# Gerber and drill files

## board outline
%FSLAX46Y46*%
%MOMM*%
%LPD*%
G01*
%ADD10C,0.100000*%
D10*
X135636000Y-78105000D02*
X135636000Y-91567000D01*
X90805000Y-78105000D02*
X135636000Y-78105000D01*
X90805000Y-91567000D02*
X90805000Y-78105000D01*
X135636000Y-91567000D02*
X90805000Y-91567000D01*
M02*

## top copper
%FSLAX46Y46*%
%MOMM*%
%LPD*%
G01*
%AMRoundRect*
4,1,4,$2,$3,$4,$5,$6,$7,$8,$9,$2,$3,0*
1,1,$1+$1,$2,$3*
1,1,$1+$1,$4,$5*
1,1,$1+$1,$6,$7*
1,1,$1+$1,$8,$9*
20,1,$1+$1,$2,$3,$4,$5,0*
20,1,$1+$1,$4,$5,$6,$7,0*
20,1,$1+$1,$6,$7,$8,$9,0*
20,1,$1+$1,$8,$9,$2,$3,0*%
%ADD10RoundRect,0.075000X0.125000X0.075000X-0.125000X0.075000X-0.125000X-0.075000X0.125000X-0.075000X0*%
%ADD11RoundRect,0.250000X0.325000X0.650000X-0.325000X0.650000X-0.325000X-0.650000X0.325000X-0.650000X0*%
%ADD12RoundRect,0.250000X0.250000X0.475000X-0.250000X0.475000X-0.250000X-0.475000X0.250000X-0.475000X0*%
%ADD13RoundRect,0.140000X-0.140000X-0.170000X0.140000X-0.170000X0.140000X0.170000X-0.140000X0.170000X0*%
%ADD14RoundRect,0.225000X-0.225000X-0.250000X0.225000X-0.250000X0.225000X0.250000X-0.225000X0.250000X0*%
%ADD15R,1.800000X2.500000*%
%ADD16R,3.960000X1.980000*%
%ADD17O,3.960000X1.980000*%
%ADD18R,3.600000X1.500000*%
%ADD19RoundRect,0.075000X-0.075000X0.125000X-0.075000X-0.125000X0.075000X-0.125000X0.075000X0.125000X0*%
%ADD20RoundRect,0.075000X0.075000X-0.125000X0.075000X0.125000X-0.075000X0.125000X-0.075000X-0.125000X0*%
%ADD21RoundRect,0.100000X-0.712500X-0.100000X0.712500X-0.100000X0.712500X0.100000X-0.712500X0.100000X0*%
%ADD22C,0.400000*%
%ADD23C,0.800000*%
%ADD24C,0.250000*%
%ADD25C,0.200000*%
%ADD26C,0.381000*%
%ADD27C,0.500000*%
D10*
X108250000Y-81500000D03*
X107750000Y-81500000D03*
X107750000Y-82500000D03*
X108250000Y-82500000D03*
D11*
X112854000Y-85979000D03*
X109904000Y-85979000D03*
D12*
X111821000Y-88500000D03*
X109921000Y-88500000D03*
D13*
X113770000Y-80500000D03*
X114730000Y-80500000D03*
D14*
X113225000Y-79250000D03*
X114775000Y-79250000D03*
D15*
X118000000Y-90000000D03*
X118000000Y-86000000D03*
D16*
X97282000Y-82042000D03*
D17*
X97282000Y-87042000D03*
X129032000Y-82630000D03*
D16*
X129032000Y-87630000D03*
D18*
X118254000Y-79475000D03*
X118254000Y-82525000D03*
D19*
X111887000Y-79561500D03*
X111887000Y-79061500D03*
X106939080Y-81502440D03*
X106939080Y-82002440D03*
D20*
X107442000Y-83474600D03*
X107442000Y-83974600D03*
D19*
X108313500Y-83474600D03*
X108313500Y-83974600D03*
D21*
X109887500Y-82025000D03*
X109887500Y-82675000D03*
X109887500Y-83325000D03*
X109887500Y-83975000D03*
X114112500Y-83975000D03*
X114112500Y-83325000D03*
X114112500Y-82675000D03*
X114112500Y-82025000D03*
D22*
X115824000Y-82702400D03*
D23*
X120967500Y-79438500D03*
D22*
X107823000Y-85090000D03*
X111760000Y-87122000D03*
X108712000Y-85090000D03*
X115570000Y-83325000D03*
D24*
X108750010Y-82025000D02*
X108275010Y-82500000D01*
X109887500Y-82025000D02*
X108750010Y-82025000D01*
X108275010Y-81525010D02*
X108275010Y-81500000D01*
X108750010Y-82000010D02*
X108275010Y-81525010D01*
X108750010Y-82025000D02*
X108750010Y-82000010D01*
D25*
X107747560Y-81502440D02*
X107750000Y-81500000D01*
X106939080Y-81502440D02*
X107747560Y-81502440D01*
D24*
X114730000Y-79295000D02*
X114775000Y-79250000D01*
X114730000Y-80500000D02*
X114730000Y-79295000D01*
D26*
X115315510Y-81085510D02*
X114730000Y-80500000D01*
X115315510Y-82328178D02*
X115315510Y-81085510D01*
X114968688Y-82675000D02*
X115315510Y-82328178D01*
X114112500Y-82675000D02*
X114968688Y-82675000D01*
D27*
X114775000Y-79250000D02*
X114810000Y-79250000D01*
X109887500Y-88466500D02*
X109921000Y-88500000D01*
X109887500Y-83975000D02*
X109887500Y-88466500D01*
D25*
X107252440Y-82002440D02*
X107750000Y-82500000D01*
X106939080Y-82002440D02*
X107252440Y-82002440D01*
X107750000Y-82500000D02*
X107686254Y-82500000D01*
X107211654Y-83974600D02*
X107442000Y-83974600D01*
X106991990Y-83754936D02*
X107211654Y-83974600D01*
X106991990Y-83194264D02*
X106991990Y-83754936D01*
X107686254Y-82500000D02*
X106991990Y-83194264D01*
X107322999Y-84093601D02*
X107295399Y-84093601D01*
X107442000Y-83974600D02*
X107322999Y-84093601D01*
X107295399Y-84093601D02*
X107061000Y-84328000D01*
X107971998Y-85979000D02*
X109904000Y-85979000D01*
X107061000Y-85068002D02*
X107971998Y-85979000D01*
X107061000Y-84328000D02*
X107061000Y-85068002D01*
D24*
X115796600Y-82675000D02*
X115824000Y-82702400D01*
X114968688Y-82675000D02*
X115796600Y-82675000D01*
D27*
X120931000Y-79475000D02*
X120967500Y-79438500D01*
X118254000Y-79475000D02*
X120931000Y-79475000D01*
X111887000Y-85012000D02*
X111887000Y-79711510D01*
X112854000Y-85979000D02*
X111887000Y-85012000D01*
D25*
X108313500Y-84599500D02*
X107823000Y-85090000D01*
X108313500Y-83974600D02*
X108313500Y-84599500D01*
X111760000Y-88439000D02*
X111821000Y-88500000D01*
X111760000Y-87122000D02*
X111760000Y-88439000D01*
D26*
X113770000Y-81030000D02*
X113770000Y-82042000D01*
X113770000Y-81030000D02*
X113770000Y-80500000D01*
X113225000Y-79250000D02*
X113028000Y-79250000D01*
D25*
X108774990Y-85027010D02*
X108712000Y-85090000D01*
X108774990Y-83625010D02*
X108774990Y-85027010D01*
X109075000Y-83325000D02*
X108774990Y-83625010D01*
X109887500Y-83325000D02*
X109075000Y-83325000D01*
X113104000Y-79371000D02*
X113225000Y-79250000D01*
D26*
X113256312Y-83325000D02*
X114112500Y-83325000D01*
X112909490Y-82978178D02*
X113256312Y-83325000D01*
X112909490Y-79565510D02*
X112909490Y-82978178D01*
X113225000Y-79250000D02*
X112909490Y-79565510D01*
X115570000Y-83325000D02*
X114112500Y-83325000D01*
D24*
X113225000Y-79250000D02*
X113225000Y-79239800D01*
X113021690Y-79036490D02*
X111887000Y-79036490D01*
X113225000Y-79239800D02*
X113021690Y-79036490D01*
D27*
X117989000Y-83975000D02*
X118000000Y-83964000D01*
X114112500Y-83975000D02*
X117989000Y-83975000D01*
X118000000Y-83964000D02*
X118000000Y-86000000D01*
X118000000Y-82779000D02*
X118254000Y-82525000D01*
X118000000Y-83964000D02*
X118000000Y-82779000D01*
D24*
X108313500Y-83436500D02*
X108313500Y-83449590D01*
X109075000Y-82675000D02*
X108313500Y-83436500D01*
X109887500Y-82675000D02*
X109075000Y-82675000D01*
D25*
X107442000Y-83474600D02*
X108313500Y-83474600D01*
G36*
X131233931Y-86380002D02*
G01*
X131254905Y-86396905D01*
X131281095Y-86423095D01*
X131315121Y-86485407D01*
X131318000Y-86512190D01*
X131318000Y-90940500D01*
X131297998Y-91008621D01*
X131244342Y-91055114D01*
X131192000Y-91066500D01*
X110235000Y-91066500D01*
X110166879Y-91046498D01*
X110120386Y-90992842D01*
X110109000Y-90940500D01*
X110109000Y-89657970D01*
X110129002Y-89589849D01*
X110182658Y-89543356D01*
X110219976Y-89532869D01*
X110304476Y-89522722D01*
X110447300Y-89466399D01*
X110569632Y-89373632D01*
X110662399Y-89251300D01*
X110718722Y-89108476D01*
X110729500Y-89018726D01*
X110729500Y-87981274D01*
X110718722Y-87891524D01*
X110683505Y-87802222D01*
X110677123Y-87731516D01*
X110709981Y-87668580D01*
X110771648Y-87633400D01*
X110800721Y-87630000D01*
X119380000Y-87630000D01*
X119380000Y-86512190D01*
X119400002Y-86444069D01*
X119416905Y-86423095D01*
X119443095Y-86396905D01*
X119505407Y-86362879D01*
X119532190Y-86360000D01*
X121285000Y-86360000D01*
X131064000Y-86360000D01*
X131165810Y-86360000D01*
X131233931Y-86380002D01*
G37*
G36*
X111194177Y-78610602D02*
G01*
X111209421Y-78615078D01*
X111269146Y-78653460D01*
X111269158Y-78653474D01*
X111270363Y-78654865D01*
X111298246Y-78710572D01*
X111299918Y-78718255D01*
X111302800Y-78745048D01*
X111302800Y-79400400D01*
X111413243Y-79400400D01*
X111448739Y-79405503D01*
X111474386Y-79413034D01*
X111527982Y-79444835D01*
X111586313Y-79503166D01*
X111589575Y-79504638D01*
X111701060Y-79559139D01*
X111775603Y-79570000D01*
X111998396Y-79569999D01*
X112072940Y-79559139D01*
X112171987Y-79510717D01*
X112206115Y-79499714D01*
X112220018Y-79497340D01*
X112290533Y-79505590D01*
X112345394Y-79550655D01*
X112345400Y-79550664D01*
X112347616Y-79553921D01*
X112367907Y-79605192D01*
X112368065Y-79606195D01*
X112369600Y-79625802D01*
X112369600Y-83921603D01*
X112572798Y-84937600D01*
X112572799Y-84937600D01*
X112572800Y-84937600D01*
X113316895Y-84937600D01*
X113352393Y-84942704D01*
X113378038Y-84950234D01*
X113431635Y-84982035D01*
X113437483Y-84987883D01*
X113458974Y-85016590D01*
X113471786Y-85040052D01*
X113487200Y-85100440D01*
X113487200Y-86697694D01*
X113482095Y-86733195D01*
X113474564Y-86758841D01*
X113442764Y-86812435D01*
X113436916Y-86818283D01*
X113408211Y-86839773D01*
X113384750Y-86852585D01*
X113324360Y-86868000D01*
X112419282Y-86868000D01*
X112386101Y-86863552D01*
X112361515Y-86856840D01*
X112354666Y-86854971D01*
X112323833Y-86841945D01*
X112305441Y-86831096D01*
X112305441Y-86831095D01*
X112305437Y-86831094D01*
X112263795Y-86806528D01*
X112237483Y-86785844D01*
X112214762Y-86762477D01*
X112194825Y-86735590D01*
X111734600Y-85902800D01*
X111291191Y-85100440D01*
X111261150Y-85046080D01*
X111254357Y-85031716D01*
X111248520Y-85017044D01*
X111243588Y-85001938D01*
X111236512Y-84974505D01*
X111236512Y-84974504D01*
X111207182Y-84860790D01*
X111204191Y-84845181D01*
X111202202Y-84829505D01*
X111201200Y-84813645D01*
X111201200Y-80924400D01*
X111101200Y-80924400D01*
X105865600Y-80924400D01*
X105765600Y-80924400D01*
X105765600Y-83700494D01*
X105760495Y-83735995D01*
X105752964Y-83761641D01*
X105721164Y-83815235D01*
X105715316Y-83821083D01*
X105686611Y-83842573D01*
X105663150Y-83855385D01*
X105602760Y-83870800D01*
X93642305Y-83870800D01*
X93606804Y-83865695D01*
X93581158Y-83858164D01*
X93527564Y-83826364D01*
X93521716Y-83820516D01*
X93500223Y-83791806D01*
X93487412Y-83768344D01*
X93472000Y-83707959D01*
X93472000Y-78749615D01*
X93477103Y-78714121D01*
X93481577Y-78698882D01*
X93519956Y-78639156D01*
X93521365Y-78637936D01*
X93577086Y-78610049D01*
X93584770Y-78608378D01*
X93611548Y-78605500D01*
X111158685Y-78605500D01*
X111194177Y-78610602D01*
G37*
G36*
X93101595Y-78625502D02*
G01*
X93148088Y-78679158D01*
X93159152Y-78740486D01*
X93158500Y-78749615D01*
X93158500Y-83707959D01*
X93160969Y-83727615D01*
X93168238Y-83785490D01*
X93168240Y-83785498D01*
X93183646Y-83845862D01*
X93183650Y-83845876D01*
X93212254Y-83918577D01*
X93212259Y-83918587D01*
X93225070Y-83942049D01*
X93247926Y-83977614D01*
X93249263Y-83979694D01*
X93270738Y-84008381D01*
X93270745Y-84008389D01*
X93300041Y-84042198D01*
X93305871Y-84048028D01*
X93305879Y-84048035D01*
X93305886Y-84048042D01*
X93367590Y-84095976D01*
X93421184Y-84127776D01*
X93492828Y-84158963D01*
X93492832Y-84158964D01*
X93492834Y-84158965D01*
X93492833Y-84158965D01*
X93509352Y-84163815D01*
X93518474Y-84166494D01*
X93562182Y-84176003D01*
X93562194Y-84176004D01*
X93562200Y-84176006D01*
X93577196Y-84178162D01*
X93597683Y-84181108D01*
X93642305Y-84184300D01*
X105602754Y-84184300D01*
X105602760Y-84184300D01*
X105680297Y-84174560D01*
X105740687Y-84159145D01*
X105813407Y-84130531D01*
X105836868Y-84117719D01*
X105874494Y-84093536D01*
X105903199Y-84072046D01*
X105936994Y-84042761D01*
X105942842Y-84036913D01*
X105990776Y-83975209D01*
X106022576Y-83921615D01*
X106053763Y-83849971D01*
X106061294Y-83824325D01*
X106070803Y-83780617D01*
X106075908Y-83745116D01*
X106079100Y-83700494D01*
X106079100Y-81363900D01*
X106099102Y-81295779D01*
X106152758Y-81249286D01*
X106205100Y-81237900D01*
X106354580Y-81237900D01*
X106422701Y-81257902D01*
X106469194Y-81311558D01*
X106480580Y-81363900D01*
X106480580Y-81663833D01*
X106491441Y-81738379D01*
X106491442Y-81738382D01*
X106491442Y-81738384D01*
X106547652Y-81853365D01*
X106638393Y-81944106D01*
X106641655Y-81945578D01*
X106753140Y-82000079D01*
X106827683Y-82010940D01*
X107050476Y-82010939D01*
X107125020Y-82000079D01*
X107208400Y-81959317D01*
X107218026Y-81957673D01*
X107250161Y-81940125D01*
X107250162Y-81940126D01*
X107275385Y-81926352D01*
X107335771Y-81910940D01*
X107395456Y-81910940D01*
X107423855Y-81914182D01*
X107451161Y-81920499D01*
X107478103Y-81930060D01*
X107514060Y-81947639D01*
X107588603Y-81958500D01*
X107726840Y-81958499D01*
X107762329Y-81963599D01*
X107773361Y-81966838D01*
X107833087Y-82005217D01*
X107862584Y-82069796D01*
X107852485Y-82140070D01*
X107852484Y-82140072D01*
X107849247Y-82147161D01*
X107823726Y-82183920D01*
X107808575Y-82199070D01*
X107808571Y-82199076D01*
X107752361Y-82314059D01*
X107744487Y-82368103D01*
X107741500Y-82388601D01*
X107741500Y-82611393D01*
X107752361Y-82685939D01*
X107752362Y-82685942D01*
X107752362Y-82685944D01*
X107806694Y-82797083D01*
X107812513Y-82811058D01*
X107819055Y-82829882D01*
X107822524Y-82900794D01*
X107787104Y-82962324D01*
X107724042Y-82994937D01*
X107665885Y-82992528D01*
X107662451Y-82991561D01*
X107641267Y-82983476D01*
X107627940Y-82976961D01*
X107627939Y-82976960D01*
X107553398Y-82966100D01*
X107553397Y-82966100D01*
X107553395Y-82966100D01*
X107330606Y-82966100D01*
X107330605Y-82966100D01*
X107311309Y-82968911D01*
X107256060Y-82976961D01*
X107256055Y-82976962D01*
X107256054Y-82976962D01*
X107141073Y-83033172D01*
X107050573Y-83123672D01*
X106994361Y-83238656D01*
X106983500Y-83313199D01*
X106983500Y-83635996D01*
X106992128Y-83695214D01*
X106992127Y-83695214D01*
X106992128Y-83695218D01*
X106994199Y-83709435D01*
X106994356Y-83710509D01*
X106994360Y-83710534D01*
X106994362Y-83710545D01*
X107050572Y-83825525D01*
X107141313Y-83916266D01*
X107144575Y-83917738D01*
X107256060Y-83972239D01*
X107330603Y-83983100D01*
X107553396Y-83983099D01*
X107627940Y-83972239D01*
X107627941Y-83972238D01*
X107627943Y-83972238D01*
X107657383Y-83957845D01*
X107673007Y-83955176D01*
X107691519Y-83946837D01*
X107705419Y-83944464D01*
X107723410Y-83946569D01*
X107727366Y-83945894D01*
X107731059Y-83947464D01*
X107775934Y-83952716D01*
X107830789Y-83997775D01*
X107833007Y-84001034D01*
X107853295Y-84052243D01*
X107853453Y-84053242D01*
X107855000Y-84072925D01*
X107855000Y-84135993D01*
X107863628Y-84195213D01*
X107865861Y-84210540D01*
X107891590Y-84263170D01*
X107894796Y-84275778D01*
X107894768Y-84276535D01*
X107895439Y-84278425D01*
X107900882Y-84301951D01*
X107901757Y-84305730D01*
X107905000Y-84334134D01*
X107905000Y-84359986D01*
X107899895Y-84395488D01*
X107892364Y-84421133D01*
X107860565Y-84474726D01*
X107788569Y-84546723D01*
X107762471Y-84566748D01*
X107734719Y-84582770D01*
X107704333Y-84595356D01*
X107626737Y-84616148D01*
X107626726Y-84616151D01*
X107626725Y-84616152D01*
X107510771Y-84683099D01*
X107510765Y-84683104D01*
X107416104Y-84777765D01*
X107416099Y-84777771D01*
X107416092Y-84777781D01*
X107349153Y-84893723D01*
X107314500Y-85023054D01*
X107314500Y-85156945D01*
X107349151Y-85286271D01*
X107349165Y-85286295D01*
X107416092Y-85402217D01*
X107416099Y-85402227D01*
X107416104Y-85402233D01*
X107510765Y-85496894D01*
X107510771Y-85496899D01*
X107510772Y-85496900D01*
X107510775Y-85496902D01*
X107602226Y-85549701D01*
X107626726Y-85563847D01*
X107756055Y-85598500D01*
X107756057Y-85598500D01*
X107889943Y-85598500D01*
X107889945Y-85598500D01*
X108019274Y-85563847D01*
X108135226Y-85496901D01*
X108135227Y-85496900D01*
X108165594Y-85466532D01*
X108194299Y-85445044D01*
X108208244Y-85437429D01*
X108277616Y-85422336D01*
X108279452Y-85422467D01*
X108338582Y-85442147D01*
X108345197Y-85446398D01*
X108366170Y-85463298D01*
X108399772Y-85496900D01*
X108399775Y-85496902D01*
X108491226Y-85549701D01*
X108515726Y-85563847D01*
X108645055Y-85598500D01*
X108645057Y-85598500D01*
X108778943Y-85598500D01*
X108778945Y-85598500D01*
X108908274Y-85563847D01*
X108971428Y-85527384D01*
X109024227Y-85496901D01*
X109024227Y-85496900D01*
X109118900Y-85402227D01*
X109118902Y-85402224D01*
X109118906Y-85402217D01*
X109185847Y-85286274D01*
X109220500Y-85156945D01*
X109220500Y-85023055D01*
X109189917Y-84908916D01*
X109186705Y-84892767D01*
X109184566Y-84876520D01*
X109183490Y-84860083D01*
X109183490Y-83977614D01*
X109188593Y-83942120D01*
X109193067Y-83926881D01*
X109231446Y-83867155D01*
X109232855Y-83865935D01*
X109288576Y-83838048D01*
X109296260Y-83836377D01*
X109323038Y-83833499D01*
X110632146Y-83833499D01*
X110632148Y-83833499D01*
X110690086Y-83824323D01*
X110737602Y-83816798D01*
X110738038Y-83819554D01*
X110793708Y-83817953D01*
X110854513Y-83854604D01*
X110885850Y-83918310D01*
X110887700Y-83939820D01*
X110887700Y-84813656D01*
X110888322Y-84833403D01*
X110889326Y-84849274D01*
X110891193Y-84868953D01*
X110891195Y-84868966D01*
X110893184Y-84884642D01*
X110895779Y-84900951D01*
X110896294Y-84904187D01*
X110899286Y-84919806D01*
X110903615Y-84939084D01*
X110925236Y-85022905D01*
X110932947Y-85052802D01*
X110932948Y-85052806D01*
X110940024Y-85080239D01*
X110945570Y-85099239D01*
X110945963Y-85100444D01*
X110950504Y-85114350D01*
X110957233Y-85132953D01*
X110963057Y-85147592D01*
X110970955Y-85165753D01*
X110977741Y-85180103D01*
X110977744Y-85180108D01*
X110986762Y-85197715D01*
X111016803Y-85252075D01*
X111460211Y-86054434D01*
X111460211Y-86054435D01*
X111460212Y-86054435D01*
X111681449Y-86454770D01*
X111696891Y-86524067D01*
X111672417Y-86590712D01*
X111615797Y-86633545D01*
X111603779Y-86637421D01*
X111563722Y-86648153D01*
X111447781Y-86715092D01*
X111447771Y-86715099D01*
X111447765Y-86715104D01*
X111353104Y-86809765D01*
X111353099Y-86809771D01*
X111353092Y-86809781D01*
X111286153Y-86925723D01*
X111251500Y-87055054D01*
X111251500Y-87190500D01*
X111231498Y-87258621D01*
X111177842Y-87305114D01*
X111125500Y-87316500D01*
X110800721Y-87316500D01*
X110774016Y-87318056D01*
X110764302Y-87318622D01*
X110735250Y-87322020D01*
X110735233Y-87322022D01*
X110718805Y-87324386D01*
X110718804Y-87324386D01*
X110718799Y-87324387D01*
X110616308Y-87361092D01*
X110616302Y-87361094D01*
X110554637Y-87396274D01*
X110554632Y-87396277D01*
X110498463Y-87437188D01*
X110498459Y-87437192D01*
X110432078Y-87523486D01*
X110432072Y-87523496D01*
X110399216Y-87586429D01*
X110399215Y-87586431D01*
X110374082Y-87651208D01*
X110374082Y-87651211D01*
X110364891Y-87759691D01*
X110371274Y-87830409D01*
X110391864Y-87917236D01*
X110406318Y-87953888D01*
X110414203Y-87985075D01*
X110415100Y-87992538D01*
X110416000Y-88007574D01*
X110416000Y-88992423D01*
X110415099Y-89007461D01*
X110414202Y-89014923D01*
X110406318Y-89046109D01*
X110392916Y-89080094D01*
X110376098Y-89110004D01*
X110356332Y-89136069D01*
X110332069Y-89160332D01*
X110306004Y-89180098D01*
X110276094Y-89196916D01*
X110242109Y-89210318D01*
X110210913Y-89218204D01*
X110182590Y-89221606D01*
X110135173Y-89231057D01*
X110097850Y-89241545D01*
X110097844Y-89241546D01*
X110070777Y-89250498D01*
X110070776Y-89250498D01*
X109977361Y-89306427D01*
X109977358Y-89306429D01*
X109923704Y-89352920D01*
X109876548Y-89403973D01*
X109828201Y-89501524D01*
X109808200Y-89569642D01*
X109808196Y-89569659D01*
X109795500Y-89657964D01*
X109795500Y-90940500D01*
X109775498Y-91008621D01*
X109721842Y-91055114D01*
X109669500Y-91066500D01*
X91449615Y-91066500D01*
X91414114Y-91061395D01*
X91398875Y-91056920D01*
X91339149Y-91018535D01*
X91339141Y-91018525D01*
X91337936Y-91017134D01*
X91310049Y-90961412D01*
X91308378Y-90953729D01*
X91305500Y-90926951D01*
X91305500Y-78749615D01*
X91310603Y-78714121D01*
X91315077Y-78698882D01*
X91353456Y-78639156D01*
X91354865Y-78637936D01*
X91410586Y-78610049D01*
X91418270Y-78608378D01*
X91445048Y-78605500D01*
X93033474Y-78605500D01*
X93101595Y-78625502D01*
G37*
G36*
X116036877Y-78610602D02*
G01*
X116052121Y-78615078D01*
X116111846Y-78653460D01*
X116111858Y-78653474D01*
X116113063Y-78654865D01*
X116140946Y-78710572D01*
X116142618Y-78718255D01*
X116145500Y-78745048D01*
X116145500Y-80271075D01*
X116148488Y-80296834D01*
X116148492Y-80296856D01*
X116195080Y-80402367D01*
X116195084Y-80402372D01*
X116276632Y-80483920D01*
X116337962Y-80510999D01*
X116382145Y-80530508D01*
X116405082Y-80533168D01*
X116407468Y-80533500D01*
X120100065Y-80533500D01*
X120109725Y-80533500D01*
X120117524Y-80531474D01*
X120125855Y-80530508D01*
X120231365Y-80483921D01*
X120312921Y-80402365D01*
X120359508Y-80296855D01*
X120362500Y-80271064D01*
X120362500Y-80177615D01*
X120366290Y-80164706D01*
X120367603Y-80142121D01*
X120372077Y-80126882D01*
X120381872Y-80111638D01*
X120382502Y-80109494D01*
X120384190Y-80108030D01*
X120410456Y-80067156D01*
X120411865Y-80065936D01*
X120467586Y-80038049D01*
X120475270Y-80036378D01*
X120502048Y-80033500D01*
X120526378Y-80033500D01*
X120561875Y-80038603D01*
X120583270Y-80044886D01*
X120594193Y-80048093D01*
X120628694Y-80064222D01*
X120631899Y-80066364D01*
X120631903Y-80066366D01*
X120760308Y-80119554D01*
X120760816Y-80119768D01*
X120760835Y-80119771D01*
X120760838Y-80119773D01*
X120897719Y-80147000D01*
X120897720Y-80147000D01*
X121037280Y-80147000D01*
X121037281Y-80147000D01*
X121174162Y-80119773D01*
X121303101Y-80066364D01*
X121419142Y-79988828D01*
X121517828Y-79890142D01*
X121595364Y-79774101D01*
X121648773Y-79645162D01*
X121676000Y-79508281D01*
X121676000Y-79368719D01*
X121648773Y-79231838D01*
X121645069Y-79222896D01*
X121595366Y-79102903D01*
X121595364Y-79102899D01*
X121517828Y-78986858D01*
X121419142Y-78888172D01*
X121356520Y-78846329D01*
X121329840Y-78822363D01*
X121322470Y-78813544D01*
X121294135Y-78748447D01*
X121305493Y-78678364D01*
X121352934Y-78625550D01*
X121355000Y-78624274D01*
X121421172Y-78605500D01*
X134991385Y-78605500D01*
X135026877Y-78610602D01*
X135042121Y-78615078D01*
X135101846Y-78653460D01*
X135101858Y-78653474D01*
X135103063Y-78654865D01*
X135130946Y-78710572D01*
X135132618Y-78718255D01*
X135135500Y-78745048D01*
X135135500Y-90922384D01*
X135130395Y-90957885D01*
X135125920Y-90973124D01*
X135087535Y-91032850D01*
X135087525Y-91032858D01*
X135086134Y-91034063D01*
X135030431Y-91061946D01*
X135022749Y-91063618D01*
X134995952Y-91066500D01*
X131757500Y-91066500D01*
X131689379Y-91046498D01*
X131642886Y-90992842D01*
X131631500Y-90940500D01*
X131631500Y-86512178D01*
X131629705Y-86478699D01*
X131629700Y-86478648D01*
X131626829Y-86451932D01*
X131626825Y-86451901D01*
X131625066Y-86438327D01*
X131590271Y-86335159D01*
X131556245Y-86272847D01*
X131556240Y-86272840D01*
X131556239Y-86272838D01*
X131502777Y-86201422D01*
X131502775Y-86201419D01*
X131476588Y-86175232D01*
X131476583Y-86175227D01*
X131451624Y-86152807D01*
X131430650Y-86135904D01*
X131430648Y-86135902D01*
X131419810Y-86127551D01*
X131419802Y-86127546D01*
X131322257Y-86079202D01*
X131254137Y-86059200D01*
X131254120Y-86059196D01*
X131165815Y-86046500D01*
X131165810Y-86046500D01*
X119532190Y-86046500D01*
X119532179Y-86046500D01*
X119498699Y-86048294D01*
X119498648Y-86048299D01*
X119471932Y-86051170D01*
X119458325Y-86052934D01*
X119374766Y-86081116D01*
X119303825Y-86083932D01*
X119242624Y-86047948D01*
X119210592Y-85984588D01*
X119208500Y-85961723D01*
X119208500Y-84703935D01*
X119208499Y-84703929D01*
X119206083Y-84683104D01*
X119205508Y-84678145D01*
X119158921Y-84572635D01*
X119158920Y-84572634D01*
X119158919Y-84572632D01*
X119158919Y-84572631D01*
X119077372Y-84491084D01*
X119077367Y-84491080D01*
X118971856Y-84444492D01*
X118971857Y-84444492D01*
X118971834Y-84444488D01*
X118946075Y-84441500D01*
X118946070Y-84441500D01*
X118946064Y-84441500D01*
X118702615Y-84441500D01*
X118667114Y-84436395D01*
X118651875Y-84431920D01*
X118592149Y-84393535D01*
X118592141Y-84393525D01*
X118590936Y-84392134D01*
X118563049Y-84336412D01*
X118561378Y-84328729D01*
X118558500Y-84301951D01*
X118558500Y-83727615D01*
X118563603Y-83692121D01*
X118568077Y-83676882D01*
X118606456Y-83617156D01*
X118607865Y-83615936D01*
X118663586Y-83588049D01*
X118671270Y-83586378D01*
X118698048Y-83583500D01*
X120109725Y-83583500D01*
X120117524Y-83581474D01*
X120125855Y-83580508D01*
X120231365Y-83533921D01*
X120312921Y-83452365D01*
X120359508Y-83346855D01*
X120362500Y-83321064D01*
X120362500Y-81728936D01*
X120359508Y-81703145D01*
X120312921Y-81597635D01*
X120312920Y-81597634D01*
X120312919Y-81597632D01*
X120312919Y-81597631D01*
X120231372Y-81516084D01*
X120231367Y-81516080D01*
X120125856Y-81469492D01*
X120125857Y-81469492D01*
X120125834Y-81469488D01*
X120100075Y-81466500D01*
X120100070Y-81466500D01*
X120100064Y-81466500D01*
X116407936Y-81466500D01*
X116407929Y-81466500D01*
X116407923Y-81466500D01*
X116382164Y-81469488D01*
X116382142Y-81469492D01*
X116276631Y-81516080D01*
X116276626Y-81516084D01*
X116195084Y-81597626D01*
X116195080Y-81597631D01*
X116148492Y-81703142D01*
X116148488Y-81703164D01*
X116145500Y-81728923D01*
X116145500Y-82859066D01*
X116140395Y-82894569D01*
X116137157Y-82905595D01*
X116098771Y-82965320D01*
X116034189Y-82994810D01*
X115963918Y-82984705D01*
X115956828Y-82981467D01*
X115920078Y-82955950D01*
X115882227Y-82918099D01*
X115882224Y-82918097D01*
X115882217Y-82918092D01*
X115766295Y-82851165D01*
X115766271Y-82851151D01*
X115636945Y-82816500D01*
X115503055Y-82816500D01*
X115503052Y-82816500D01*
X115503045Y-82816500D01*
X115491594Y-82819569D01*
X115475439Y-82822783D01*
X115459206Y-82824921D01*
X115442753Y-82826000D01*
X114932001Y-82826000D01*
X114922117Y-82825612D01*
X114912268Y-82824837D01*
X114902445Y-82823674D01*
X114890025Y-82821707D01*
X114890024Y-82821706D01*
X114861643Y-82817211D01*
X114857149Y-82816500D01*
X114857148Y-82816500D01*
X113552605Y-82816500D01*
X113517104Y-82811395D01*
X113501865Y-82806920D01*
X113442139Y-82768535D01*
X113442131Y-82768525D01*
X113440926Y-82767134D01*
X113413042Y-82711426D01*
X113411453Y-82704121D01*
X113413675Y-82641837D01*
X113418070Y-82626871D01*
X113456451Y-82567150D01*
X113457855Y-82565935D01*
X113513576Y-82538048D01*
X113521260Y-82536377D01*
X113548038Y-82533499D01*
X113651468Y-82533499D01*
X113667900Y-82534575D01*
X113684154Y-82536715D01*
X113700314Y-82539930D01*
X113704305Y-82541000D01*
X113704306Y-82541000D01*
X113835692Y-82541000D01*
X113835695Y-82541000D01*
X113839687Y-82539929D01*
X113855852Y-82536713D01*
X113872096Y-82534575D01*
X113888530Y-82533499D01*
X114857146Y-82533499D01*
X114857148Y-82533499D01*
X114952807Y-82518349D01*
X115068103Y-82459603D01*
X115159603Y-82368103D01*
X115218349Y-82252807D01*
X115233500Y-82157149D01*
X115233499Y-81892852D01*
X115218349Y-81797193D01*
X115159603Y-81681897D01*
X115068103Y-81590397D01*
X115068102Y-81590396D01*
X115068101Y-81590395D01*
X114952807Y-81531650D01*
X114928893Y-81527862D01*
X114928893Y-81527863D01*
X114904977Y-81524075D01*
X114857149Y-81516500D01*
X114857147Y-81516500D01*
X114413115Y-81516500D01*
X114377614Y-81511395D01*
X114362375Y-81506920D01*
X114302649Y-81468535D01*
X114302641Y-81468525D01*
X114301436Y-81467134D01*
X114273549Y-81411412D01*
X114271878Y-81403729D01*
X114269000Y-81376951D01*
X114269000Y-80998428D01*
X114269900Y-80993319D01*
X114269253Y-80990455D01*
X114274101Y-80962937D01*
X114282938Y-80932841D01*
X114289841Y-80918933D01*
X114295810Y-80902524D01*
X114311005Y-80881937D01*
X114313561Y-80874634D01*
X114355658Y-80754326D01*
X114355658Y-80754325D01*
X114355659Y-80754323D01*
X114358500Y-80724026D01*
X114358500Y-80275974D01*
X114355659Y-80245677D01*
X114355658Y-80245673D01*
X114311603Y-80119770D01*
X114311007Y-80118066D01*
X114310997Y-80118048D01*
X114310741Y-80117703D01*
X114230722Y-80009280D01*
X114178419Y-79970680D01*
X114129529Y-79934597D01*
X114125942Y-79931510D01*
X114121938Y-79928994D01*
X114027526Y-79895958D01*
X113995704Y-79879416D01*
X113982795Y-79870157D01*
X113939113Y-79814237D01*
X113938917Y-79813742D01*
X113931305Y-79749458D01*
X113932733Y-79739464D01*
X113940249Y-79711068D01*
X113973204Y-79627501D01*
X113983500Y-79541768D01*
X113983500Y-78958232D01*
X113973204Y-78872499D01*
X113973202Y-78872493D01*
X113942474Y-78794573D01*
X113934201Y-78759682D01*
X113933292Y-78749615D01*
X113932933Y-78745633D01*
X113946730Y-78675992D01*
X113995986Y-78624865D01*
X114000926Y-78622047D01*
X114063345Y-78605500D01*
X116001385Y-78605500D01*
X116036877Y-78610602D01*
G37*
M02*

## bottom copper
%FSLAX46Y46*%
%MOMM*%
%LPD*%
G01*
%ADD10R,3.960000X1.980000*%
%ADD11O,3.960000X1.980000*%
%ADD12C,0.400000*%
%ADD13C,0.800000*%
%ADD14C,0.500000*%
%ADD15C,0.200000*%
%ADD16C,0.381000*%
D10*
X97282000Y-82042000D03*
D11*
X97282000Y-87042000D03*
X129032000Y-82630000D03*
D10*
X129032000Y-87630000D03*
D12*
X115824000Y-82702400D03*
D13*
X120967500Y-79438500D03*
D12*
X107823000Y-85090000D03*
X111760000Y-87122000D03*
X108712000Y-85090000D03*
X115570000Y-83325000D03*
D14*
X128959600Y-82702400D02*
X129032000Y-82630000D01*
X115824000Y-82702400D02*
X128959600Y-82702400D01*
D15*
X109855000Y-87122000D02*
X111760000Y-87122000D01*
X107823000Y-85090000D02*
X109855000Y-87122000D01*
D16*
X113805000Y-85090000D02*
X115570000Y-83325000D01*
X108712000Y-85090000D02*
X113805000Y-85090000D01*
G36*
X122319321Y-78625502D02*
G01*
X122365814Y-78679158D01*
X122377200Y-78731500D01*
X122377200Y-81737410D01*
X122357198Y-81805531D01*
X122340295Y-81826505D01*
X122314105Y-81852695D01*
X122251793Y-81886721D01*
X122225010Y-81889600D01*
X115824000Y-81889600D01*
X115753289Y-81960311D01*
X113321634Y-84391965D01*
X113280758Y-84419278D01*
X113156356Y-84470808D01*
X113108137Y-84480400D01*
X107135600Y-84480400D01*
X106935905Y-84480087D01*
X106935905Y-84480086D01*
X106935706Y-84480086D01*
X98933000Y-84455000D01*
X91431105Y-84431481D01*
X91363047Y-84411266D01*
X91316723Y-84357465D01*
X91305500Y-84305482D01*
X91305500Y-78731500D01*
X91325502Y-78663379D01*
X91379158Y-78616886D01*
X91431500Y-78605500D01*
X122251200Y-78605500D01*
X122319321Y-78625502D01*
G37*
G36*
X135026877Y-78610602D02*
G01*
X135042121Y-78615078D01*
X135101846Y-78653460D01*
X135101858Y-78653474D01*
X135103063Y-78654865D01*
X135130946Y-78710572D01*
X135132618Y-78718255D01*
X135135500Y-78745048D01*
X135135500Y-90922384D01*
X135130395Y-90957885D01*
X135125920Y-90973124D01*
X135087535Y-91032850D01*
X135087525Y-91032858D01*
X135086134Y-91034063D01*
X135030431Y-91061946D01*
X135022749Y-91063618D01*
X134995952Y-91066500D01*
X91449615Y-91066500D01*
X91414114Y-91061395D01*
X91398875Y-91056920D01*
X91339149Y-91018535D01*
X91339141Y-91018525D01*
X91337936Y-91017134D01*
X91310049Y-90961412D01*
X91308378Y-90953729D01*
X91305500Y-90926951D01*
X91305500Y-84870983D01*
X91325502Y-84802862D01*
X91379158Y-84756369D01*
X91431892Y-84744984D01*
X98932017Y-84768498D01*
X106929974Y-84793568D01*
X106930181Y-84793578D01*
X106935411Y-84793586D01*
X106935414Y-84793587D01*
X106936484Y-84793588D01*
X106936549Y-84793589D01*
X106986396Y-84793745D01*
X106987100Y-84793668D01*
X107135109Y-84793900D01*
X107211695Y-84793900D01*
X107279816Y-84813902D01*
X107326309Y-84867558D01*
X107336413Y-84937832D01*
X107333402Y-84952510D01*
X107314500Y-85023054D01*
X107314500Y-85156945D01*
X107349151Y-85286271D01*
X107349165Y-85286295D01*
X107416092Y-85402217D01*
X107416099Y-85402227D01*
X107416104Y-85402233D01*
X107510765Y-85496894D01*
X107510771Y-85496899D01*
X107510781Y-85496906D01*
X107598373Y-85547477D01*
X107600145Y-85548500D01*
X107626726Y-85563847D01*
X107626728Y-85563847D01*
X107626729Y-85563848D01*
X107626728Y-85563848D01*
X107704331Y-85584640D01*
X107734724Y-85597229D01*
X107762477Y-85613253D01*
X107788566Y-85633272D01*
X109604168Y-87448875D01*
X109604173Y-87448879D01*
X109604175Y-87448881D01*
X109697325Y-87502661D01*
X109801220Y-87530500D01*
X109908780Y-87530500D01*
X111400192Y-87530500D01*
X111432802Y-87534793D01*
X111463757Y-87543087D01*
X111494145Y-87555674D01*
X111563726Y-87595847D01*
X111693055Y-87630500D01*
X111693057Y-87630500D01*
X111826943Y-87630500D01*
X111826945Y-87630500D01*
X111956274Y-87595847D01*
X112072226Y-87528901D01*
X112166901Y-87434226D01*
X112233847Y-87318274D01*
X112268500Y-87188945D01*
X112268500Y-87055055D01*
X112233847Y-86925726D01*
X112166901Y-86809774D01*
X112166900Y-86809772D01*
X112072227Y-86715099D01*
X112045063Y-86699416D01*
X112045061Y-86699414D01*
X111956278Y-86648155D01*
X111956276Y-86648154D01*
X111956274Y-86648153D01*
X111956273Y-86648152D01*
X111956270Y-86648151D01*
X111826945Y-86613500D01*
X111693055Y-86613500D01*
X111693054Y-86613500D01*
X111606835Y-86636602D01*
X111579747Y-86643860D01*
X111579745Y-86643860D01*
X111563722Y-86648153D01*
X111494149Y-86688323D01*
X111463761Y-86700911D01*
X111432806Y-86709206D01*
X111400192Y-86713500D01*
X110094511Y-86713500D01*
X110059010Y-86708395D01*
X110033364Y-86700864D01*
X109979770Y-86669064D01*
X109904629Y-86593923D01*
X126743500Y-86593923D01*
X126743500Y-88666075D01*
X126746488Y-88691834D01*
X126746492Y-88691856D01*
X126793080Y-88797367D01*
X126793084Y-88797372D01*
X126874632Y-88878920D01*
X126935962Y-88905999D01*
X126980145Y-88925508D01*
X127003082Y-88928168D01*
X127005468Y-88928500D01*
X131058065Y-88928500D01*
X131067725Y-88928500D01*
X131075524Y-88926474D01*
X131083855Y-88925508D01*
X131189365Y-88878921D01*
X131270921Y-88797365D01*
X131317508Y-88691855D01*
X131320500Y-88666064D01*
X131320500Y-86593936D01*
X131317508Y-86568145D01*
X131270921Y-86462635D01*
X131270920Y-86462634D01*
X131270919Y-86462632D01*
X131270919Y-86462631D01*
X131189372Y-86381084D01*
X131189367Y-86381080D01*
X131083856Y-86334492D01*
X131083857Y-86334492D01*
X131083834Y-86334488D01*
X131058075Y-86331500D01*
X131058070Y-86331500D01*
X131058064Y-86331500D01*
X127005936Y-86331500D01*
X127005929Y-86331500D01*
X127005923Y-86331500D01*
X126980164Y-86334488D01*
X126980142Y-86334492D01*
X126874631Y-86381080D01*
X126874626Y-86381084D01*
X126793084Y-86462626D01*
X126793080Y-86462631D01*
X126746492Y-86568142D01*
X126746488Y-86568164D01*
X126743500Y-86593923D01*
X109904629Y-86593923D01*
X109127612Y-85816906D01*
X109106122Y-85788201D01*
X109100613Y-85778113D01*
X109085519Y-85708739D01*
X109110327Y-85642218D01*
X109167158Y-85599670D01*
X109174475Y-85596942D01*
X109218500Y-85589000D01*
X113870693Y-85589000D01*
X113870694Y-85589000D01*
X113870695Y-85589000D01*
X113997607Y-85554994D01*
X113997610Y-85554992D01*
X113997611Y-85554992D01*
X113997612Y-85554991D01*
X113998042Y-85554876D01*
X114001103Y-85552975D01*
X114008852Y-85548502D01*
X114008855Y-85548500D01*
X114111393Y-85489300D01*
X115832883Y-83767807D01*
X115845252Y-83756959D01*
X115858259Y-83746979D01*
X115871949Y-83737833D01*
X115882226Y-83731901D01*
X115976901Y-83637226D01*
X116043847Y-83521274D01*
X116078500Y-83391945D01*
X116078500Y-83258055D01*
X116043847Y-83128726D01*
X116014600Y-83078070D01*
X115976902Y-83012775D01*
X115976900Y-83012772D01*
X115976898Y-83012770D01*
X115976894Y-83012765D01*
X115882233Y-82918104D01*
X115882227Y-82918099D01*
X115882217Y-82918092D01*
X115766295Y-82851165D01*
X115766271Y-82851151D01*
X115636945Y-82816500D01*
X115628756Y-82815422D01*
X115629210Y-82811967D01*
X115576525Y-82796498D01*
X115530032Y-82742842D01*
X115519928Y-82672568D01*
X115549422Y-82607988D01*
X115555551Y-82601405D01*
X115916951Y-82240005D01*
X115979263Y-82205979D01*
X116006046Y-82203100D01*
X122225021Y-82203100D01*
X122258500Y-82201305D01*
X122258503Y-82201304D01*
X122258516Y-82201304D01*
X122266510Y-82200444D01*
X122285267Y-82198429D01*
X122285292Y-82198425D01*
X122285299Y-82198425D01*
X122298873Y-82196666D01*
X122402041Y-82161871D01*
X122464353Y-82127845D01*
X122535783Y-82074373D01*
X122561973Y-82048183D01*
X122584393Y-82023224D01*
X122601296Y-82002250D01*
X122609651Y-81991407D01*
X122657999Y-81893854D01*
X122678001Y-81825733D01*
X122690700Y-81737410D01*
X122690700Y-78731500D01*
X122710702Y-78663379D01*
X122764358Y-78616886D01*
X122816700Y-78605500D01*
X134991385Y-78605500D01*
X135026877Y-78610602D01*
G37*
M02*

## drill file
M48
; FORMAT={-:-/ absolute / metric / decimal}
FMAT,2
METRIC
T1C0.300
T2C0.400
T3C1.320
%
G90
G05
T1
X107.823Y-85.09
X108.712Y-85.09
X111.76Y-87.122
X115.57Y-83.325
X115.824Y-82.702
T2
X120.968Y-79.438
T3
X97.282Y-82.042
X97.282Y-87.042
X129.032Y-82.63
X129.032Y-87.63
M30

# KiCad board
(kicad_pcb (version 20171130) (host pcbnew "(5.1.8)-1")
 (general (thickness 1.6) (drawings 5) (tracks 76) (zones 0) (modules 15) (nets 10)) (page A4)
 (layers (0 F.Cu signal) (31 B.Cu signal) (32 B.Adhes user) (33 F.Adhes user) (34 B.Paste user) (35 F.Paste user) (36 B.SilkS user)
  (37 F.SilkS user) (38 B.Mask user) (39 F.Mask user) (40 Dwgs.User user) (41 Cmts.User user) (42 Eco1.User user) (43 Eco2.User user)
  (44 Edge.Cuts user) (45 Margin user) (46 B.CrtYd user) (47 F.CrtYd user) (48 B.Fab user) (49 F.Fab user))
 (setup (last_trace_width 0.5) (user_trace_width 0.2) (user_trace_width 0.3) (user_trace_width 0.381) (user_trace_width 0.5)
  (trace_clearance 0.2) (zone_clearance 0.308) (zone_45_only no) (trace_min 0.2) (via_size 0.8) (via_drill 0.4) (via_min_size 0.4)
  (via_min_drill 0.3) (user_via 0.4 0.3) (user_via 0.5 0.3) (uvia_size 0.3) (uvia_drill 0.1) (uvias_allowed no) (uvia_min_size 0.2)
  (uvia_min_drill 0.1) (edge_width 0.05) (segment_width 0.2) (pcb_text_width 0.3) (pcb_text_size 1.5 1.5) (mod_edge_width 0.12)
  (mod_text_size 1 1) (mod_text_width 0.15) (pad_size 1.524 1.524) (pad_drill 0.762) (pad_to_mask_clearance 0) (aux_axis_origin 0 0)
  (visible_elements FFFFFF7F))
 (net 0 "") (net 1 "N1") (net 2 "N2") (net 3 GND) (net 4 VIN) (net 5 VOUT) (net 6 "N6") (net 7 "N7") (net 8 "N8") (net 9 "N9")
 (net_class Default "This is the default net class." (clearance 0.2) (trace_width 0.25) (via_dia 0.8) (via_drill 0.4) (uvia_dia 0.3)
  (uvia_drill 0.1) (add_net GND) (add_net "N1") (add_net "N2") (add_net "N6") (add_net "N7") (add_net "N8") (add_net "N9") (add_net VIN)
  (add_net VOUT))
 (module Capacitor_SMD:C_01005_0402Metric (layer F.Cu) (at 108 81.5 180)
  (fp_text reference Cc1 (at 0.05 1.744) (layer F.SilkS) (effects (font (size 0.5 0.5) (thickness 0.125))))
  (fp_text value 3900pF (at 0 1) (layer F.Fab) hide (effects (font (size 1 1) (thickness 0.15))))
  (pad "" smd roundrect (at -0.275 0 180) (size 0.27 0.27) (layers F.Paste) (roundrect_rratio 0.25))
  (pad "" smd roundrect (at 0.275 0 180) (size 0.27 0.27) (layers F.Paste) (roundrect_rratio 0.25))
  (pad 1 smd roundrect (at -0.25 0 180) (size 0.4 0.3) (layers F.Cu F.Mask) (roundrect_rratio 0.25) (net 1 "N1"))
  (pad 2 smd roundrect (at 0.25 0 180) (size 0.4 0.3) (layers F.Cu F.Mask) (roundrect_rratio 0.25) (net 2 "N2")))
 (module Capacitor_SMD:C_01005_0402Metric (layer F.Cu) (at 108 82.5 180)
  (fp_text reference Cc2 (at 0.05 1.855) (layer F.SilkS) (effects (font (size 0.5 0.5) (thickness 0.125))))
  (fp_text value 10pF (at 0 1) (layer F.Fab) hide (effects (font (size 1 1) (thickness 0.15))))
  (pad 2 smd roundrect (at 0.25 0 180) (size 0.4 0.3) (layers F.Cu F.Mask) (roundrect_rratio 0.25) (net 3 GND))
  (pad 1 smd roundrect (at -0.25 0 180) (size 0.4 0.3) (layers F.Cu F.Mask) (roundrect_rratio 0.25) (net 1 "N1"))
  (pad "" smd roundrect (at 0.275 0 180) (size 0.27 0.27) (layers F.Paste) (roundrect_rratio 0.25))
  (pad "" smd roundrect (at -0.275 0 180) (size 0.27 0.27) (layers F.Paste) (roundrect_rratio 0.25)))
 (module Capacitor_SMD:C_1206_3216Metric (layer F.Cu) (at 111.379 85.979 180)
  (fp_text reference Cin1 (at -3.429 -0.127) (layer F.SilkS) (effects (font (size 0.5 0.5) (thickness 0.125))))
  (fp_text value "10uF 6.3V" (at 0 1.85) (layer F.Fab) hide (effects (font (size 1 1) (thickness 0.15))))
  (pad 1 smd roundrect (at -1.475 0 180) (size 1.15 1.8) (layers F.Cu F.Paste F.Mask) (roundrect_rratio 0.217391) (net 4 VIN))
  (pad 2 smd roundrect (at 1.475 0 180) (size 1.15 1.8) (layers F.Cu F.Paste F.Mask) (roundrect_rratio 0.217391) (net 3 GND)))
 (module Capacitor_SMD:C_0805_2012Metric (layer F.Cu) (at 110.871 88.5 180)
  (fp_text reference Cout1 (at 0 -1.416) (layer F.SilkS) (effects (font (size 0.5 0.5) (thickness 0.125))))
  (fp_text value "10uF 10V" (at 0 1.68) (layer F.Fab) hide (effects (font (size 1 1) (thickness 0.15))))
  (pad 1 smd roundrect (at -0.95 0 180) (size 1 1.45) (layers F.Cu F.Paste F.Mask) (roundrect_rratio 0.25) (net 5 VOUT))
  (pad 2 smd roundrect (at 0.95 0 180) (size 1 1.45) (layers F.Cu F.Paste F.Mask) (roundrect_rratio 0.25) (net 3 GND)))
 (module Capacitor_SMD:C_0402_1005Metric (layer F.Cu) (at 114.25 80.5)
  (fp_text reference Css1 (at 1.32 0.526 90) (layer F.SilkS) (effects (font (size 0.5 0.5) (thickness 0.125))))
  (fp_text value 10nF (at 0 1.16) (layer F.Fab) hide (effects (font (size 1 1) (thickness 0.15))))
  (pad 1 smd roundrect (at -0.48 0) (size 0.56 0.62) (layers F.Cu F.Paste F.Mask) (roundrect_rratio 0.25) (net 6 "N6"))
  (pad 2 smd roundrect (at 0.48 0) (size 0.56 0.62) (layers F.Cu F.Paste F.Mask) (roundrect_rratio 0.25) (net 3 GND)))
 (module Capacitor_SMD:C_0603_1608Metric (layer F.Cu) (at 114 79.25)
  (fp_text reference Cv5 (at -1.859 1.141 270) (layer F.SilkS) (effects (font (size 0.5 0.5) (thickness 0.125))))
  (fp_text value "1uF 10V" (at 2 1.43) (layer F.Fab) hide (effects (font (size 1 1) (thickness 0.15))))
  (pad 1 smd roundrect (at -0.775 0) (size 0.9 0.95) (layers F.Cu F.Paste F.Mask) (roundrect_rratio 0.25) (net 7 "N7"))
  (pad 2 smd roundrect (at 0.775 0) (size 0.9 0.95) (layers F.Cu F.Paste F.Mask) (roundrect_rratio 0.25) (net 3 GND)))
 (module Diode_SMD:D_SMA (layer F.Cu) (at 118 88 90)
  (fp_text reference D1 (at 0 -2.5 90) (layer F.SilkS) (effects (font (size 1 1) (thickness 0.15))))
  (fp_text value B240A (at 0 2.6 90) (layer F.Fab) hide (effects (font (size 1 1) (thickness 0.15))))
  (pad 1 smd rect (at -2 0 90) (size 2.5 1.8) (layers F.Cu F.Paste F.Mask) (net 5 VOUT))
  (pad 2 smd rect (at 2 0 90) (size 2.5 1.8) (layers F.Cu F.Paste F.Mask) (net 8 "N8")))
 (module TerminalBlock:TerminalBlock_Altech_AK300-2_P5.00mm (layer F.Cu) (at 97.282 82.042 270)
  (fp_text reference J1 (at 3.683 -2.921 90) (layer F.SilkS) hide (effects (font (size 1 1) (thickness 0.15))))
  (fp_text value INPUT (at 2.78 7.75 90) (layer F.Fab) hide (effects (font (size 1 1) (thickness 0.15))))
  (pad 1 thru_hole rect (at 0 0 270) (size 1.98 3.96) (drill 1.32) (layers *.Cu *.Mask) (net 4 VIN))
  (pad 2 thru_hole oval (at 5 0 270) (size 1.98 3.96) (drill 1.32) (layers *.Cu *.Mask) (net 3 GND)))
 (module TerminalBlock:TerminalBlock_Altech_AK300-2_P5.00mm (layer F.Cu) (at 129.032 87.63 90)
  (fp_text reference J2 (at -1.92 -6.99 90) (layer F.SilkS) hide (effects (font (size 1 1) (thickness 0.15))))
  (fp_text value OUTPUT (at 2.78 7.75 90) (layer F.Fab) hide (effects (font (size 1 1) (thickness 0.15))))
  (pad 2 thru_hole oval (at 5 0 90) (size 1.98 3.96) (drill 1.32) (layers *.Cu *.Mask) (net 3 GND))
  (pad 1 thru_hole rect (at 0 0 90) (size 1.98 3.96) (drill 1.32) (layers *.Cu *.Mask) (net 5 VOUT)))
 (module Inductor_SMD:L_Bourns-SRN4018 (layer F.Cu) (at 118.254 81 270)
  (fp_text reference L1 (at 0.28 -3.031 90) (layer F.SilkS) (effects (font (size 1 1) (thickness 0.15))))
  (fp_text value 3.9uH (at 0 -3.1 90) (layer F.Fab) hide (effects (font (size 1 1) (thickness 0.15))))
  (pad 1 smd rect (at -1.525 0 270) (size 1.5 3.6) (layers F.Cu F.Paste F.Mask) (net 4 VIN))
  (pad 2 smd rect (at 1.525 0 270) (size 1.5 3.6) (layers F.Cu F.Paste F.Mask) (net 8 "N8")))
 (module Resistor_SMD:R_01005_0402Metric (layer F.Cu) (at 111.887 79.3115 270)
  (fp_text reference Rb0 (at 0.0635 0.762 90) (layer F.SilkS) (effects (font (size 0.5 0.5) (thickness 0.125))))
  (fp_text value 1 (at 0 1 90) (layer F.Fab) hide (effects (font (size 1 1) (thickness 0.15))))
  (pad 2 smd roundrect (at 0.25 0 270) (size 0.4 0.3) (layers F.Cu F.Mask) (roundrect_rratio 0.25) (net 4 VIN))
  (pad 1 smd roundrect (at -0.25 0 270) (size 0.4 0.3) (layers F.Cu F.Mask) (roundrect_rratio 0.25) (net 7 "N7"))
  (pad "" smd roundrect (at 0.275 0 270) (size 0.27 0.27) (layers F.Paste) (roundrect_rratio 0.25))
  (pad "" smd roundrect (at -0.275 0 270) (size 0.27 0.27) (layers F.Paste) (roundrect_rratio 0.25)))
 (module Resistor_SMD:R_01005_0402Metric (layer F.Cu) (at 106.93908 81.75244 270)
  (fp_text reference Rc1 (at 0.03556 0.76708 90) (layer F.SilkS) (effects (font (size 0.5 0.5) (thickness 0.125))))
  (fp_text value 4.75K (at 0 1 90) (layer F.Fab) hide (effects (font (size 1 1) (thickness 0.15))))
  (pad "" smd roundrect (at -0.275 0 270) (size 0.27 0.27) (layers F.Paste) (roundrect_rratio 0.25))
  (pad "" smd roundrect (at 0.275 0 270) (size 0.27 0.27) (layers F.Paste) (roundrect_rratio 0.25))
  (pad 1 smd roundrect (at -0.25 0 270) (size 0.4 0.3) (layers F.Cu F.Mask) (roundrect_rratio 0.25) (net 2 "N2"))
  (pad 2 smd roundrect (at 0.25 0 270) (size 0.4 0.3) (layers F.Cu F.Mask) (roundrect_rratio 0.25) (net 3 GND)))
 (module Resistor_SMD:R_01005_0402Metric (layer F.Cu) (at 107.442 83.7246 90)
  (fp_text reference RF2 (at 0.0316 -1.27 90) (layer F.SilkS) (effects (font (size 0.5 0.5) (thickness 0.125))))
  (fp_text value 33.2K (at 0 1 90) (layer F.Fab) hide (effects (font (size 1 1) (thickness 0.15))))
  (pad 2 smd roundrect (at 0.25 0 90) (size 0.4 0.3) (layers F.Cu F.Mask) (roundrect_rratio 0.25) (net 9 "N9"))
  (pad 1 smd roundrect (at -0.25 0 90) (size 0.4 0.3) (layers F.Cu F.Mask) (roundrect_rratio 0.25) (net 3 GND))
  (pad "" smd roundrect (at 0.275 0 90) (size 0.27 0.27) (layers F.Paste) (roundrect_rratio 0.25))
  (pad "" smd roundrect (at -0.275 0 90) (size 0.27 0.27) (layers F.Paste) (roundrect_rratio 0.25)))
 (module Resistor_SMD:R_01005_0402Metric (layer F.Cu) (at 108.3135 83.7246 270)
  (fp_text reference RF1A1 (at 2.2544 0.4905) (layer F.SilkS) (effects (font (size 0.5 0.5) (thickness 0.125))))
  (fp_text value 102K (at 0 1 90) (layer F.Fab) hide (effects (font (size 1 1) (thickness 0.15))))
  (pad "" smd roundrect (at -0.275 0 270) (size 0.27 0.27) (layers F.Paste) (roundrect_rratio 0.25))
  (pad "" smd roundrect (at 0.275 0 270) (size 0.27 0.27) (layers F.Paste) (roundrect_rratio 0.25))
  (pad 1 smd roundrect (at -0.25 0 270) (size 0.4 0.3) (layers F.Cu F.Mask) (roundrect_rratio 0.25) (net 9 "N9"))
  (pad 2 smd roundrect (at 0.25 0 270) (size 0.4 0.3) (layers F.Cu F.Mask) (roundrect_rratio 0.25) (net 5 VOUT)))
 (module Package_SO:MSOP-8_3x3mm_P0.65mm (layer F.Cu) (at 112 83)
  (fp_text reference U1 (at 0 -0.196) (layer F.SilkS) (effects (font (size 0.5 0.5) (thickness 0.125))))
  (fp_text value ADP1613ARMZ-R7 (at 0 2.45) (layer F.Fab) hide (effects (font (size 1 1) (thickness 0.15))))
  (pad 1 smd roundrect (at -2.1125 -0.975) (size 1.625 0.4) (layers F.Cu F.Paste F.Mask) (roundrect_rratio 0.25) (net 1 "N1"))
  (pad 2 smd roundrect (at -2.1125 -0.325) (size 1.625 0.4) (layers F.Cu F.Paste F.Mask) (roundrect_rratio 0.25) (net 9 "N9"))
  (pad 3 smd roundrect (at -2.1125 0.325) (size 1.625 0.4) (layers F.Cu F.Paste F.Mask) (roundrect_rratio 0.25) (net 7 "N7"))
  (pad 4 smd roundrect (at -2.1125 0.975) (size 1.625 0.4) (layers F.Cu F.Paste F.Mask) (roundrect_rratio 0.25) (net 3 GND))
  (pad 5 smd roundrect (at 2.1125 0.975) (size 1.625 0.4) (layers F.Cu F.Paste F.Mask) (roundrect_rratio 0.25) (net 8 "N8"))
  (pad 6 smd roundrect (at 2.1125 0.325) (size 1.625 0.4) (layers F.Cu F.Paste F.Mask) (roundrect_rratio 0.25) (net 7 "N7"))
  (pad 7 smd roundrect (at 2.1125 -0.325) (size 1.625 0.4) (layers F.Cu F.Paste F.Mask) (roundrect_rratio 0.25) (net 3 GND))
  (pad 8 smd roundrect (at 2.1125 -0.975) (size 1.625 0.4) (layers F.Cu F.Paste F.Mask) (roundrect_rratio 0.25) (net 6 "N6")))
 (gr_line (start 135.636 78.105) (end 135.636 91.567) (layer Edge.Cuts) (width 0.1))
 (gr_line (start 90.805 78.105) (end 135.636 78.105) (layer Edge.Cuts) (width 0.1))
 (gr_line (start 90.805 91.567) (end 90.805 78.105) (layer Edge.Cuts) (width 0.1))
 (gr_line (start 135.636 91.567) (end 90.805 91.567) (layer Edge.Cuts) (width 0.1))
 (segment (start 108.75001 82.025) (end 108.27501 82.5) (width 0.25) (layer F.Cu) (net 1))
 (segment (start 109.8875 82.025) (end 108.75001 82.025) (width 0.25) (layer F.Cu) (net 1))
 (segment (start 108.27501 81.52501) (end 108.27501 81.5) (width 0.25) (layer F.Cu) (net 1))
 (segment (start 108.75001 82.00001) (end 108.27501 81.52501) (width 0.25) (layer F.Cu) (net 1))
 (segment (start 108.75001 82.025) (end 108.75001 82.00001) (width 0.25) (layer F.Cu) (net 1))
 (segment (start 107.74756 81.50244) (end 107.75 81.5) (width 0.2) (layer F.Cu) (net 2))
 (segment (start 106.93908 81.50244) (end 107.74756 81.50244) (width 0.2) (layer F.Cu) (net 2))
 (segment (start 114.73 79.295) (end 114.775 79.25) (width 0.25) (layer F.Cu) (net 3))
 (segment (start 114.73 80.5) (end 114.73 79.295) (width 0.25) (layer F.Cu) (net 3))
 (segment (start 115.31551 81.08551) (end 114.73 80.5) (width 0.381) (layer F.Cu) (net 3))
 (segment (start 115.31551 82.328178) (end 115.31551 81.08551) (width 0.381) (layer F.Cu) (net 3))
 (segment (start 114.968688 82.675) (end 115.31551 82.328178) (width 0.381) (layer F.Cu) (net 3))
 (segment (start 114.1125 82.675) (end 114.968688 82.675) (width 0.381) (layer F.Cu) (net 3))
 (segment (start 114.775 79.25) (end 114.81 79.25) (width 0.5) (layer F.Cu) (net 3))
 (segment (start 109.8875 88.4665) (end 109.921 88.5) (width 0.5) (layer F.Cu) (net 3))
 (segment (start 109.8875 83.975) (end 109.8875 88.4665) (width 0.5) (layer F.Cu) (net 3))
 (segment (start 107.25244 82.00244) (end 107.75 82.5) (width 0.2) (layer F.Cu) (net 3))
 (segment (start 106.93908 82.00244) (end 107.25244 82.00244) (width 0.2) (layer F.Cu) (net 3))
 (segment (start 107.75 82.5) (end 107.686254 82.5) (width 0.2) (layer F.Cu) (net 3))
 (segment (start 107.211654 83.9746) (end 107.442 83.9746) (width 0.2) (layer F.Cu) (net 3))
 (segment (start 106.99199 83.754936) (end 107.211654 83.9746) (width 0.2) (layer F.Cu) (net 3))
 (segment (start 106.99199 83.194264) (end 106.99199 83.754936) (width 0.2) (layer F.Cu) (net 3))
 (segment (start 107.686254 82.5) (end 106.99199 83.194264) (width 0.2) (layer F.Cu) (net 3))
 (segment (start 107.322999 84.093601) (end 107.295399 84.093601) (width 0.2) (layer F.Cu) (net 3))
 (segment (start 107.442 83.9746) (end 107.322999 84.093601) (width 0.2) (layer F.Cu) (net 3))
 (segment (start 107.295399 84.093601) (end 107.061 84.328) (width 0.2) (layer F.Cu) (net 3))
 (segment (start 107.971998 85.979) (end 109.904 85.979) (width 0.2) (layer F.Cu) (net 3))
 (segment (start 107.061 85.068002) (end 107.971998 85.979) (width 0.2) (layer F.Cu) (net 3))
 (segment (start 107.061 84.328) (end 107.061 85.068002) (width 0.2) (layer F.Cu) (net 3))
 (segment (start 115.7966 82.675) (end 115.824 82.7024) (width 0.25) (layer F.Cu) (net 3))
 (via (at 115.824 82.7024) (size 0.4) (drill 0.3) (layers F.Cu B.Cu) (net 3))
 (segment (start 114.968688 82.675) (end 115.7966 82.675) (width 0.25) (layer F.Cu) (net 3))
 (segment (start 128.9596 82.7024) (end 129.032 82.63) (width 0.5) (layer B.Cu) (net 3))
 (segment (start 115.824 82.7024) (end 128.9596 82.7024) (width 0.5) (layer B.Cu) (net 3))
 (via (at 120.9675 79.4385) (size 0.8) (drill 0.4) (layers F.Cu B.Cu) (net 4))
 (segment (start 120.931 79.475) (end 120.9675 79.4385) (width 0.5) (layer F.Cu) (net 4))
 (segment (start 118.254 79.475) (end 120.931 79.475) (width 0.5) (layer F.Cu) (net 4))
 (segment (start 111.887 85.012) (end 111.887 79.71151) (width 0.5) (layer F.Cu) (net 4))
 (segment (start 112.854 85.979) (end 111.887 85.012) (width 0.5) (layer F.Cu) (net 4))
 (via (at 107.823 85.09) (size 0.4) (drill 0.3) (layers F.Cu B.Cu) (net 5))
 (segment (start 108.3135 84.5995) (end 107.823 85.09) (width 0.2) (layer F.Cu) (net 5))
 (segment (start 108.3135 83.9746) (end 108.3135 84.5995) (width 0.2) (layer F.Cu) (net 5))
 (via (at 111.76 87.122) (size 0.4) (drill 0.3) (layers F.Cu B.Cu) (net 5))
 (segment (start 109.855 87.122) (end 111.76 87.122) (width 0.2) (layer B.Cu) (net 5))
 (segment (start 107.823 85.09) (end 109.855 87.122) (width 0.2) (layer B.Cu) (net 5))
 (segment (start 111.76 88.439) (end 111.821 88.5) (width 0.2) (layer F.Cu) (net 5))
 (segment (start 111.76 87.122) (end 111.76 88.439) (width 0.2) (layer F.Cu) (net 5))
 (segment (start 113.77 81.03) (end 113.77 82.042) (width 0.381) (layer F.Cu) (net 6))
 (segment (start 113.77 81.03) (end 113.77 80.5) (width 0.381) (layer F.Cu) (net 6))
 (segment (start 113.225 79.25) (end 113.028 79.25) (width 0.381) (layer F.Cu) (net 7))
 (via (at 108.712 85.09) (size 0.4) (drill 0.3) (layers F.Cu B.Cu) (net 7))
 (segment (start 108.77499 85.02701) (end 108.712 85.09) (width 0.2) (layer F.Cu) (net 7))
 (segment (start 108.77499 83.62501) (end 108.77499 85.02701) (width 0.2) (layer F.Cu) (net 7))
 (segment (start 109.075 83.325) (end 108.77499 83.62501) (width 0.2) (layer F.Cu) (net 7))
 (segment (start 109.8875 83.325) (end 109.075 83.325) (width 0.2) (layer F.Cu) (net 7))
 (segment (start 113.104 79.371) (end 113.225 79.25) (width 0.2) (layer F.Cu) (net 7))
 (segment (start 113.256312 83.325) (end 114.1125 83.325) (width 0.381) (layer F.Cu) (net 7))
 (segment (start 112.90949 82.978178) (end 113.256312 83.325) (width 0.381) (layer F.Cu) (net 7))
 (segment (start 112.90949 79.56551) (end 112.90949 82.978178) (width 0.381) (layer F.Cu) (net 7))
 (segment (start 113.225 79.25) (end 112.90949 79.56551) (width 0.381) (layer F.Cu) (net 7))
 (via (at 115.57 83.325) (size 0.4) (drill 0.3) (layers F.Cu B.Cu) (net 7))
 (segment (start 113.805 85.09) (end 115.57 83.325) (width 0.381) (layer B.Cu) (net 7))
 (segment (start 108.712 85.09) (end 113.805 85.09) (width 0.381) (layer B.Cu) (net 7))
 (segment (start 115.57 83.325) (end 114.1125 83.325) (width 0.381) (layer F.Cu) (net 7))
 (segment (start 113.225 79.25) (end 113.225 79.2398) (width 0.25) (layer F.Cu) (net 7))
 (segment (start 113.02169 79.03649) (end 111.887 79.03649) (width 0.25) (layer F.Cu) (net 7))
 (segment (start 113.225 79.2398) (end 113.02169 79.03649) (width 0.25) (layer F.Cu) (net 7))
 (segment (start 117.989 83.975) (end 118 83.964) (width 0.5) (layer F.Cu) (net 8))
 (segment (start 114.1125 83.975) (end 117.989 83.975) (width 0.5) (layer F.Cu) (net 8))
 (segment (start 118 83.964) (end 118 86) (width 0.5) (layer F.Cu) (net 8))
 (segment (start 118 82.779) (end 118.254 82.525) (width 0.5) (layer F.Cu) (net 8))
 (segment (start 118 83.964) (end 118 82.779) (width 0.5) (layer F.Cu) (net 8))
 (segment (start 108.3135 83.4365) (end 108.3135 83.44959) (width 0.25) (layer F.Cu) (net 9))
 (segment (start 109.075 82.675) (end 108.3135 83.4365) (width 0.25) (layer F.Cu) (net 9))
 (segment (start 109.8875 82.675) (end 109.075 82.675) (width 0.25) (layer F.Cu) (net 9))
 (segment (start 107.442 83.4746) (end 108.3135 83.4746) (width 0.2) (layer F.Cu) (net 9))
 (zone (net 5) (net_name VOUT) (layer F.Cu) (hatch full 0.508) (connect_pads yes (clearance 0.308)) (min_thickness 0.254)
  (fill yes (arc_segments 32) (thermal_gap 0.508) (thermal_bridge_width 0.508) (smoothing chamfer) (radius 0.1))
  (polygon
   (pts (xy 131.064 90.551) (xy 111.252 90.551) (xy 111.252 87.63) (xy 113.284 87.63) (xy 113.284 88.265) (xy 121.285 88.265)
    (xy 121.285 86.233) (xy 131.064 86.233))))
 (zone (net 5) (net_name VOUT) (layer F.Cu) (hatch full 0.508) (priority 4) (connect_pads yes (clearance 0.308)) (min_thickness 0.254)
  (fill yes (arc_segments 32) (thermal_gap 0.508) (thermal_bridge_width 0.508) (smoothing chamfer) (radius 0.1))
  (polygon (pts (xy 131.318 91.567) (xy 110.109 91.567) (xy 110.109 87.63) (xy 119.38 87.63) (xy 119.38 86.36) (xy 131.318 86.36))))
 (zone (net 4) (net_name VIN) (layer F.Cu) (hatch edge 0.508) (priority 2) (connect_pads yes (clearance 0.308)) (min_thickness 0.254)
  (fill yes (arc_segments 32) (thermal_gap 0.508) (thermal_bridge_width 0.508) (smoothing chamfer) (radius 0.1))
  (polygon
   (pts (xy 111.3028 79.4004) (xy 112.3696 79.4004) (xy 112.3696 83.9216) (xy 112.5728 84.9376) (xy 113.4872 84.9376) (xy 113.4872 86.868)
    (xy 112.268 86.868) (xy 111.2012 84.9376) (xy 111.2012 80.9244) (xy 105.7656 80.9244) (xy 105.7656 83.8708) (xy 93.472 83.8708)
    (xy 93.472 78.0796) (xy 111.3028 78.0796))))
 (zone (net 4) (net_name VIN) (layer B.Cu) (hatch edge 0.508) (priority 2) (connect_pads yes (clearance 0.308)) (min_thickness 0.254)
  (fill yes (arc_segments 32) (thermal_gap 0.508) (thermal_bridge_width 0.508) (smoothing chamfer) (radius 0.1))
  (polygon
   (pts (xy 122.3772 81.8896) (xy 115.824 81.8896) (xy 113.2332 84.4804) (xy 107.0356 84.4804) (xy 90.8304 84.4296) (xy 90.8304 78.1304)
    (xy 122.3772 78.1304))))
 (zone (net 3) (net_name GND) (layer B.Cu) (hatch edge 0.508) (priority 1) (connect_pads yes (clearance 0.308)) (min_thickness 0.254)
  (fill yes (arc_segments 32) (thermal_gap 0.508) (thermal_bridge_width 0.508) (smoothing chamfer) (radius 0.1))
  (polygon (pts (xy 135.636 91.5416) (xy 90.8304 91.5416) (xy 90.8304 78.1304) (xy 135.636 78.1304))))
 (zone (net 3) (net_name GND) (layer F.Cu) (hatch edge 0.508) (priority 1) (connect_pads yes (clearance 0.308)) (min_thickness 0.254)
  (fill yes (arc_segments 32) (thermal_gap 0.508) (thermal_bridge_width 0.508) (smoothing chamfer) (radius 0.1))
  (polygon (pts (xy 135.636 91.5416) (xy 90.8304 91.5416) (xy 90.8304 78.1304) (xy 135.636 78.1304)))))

